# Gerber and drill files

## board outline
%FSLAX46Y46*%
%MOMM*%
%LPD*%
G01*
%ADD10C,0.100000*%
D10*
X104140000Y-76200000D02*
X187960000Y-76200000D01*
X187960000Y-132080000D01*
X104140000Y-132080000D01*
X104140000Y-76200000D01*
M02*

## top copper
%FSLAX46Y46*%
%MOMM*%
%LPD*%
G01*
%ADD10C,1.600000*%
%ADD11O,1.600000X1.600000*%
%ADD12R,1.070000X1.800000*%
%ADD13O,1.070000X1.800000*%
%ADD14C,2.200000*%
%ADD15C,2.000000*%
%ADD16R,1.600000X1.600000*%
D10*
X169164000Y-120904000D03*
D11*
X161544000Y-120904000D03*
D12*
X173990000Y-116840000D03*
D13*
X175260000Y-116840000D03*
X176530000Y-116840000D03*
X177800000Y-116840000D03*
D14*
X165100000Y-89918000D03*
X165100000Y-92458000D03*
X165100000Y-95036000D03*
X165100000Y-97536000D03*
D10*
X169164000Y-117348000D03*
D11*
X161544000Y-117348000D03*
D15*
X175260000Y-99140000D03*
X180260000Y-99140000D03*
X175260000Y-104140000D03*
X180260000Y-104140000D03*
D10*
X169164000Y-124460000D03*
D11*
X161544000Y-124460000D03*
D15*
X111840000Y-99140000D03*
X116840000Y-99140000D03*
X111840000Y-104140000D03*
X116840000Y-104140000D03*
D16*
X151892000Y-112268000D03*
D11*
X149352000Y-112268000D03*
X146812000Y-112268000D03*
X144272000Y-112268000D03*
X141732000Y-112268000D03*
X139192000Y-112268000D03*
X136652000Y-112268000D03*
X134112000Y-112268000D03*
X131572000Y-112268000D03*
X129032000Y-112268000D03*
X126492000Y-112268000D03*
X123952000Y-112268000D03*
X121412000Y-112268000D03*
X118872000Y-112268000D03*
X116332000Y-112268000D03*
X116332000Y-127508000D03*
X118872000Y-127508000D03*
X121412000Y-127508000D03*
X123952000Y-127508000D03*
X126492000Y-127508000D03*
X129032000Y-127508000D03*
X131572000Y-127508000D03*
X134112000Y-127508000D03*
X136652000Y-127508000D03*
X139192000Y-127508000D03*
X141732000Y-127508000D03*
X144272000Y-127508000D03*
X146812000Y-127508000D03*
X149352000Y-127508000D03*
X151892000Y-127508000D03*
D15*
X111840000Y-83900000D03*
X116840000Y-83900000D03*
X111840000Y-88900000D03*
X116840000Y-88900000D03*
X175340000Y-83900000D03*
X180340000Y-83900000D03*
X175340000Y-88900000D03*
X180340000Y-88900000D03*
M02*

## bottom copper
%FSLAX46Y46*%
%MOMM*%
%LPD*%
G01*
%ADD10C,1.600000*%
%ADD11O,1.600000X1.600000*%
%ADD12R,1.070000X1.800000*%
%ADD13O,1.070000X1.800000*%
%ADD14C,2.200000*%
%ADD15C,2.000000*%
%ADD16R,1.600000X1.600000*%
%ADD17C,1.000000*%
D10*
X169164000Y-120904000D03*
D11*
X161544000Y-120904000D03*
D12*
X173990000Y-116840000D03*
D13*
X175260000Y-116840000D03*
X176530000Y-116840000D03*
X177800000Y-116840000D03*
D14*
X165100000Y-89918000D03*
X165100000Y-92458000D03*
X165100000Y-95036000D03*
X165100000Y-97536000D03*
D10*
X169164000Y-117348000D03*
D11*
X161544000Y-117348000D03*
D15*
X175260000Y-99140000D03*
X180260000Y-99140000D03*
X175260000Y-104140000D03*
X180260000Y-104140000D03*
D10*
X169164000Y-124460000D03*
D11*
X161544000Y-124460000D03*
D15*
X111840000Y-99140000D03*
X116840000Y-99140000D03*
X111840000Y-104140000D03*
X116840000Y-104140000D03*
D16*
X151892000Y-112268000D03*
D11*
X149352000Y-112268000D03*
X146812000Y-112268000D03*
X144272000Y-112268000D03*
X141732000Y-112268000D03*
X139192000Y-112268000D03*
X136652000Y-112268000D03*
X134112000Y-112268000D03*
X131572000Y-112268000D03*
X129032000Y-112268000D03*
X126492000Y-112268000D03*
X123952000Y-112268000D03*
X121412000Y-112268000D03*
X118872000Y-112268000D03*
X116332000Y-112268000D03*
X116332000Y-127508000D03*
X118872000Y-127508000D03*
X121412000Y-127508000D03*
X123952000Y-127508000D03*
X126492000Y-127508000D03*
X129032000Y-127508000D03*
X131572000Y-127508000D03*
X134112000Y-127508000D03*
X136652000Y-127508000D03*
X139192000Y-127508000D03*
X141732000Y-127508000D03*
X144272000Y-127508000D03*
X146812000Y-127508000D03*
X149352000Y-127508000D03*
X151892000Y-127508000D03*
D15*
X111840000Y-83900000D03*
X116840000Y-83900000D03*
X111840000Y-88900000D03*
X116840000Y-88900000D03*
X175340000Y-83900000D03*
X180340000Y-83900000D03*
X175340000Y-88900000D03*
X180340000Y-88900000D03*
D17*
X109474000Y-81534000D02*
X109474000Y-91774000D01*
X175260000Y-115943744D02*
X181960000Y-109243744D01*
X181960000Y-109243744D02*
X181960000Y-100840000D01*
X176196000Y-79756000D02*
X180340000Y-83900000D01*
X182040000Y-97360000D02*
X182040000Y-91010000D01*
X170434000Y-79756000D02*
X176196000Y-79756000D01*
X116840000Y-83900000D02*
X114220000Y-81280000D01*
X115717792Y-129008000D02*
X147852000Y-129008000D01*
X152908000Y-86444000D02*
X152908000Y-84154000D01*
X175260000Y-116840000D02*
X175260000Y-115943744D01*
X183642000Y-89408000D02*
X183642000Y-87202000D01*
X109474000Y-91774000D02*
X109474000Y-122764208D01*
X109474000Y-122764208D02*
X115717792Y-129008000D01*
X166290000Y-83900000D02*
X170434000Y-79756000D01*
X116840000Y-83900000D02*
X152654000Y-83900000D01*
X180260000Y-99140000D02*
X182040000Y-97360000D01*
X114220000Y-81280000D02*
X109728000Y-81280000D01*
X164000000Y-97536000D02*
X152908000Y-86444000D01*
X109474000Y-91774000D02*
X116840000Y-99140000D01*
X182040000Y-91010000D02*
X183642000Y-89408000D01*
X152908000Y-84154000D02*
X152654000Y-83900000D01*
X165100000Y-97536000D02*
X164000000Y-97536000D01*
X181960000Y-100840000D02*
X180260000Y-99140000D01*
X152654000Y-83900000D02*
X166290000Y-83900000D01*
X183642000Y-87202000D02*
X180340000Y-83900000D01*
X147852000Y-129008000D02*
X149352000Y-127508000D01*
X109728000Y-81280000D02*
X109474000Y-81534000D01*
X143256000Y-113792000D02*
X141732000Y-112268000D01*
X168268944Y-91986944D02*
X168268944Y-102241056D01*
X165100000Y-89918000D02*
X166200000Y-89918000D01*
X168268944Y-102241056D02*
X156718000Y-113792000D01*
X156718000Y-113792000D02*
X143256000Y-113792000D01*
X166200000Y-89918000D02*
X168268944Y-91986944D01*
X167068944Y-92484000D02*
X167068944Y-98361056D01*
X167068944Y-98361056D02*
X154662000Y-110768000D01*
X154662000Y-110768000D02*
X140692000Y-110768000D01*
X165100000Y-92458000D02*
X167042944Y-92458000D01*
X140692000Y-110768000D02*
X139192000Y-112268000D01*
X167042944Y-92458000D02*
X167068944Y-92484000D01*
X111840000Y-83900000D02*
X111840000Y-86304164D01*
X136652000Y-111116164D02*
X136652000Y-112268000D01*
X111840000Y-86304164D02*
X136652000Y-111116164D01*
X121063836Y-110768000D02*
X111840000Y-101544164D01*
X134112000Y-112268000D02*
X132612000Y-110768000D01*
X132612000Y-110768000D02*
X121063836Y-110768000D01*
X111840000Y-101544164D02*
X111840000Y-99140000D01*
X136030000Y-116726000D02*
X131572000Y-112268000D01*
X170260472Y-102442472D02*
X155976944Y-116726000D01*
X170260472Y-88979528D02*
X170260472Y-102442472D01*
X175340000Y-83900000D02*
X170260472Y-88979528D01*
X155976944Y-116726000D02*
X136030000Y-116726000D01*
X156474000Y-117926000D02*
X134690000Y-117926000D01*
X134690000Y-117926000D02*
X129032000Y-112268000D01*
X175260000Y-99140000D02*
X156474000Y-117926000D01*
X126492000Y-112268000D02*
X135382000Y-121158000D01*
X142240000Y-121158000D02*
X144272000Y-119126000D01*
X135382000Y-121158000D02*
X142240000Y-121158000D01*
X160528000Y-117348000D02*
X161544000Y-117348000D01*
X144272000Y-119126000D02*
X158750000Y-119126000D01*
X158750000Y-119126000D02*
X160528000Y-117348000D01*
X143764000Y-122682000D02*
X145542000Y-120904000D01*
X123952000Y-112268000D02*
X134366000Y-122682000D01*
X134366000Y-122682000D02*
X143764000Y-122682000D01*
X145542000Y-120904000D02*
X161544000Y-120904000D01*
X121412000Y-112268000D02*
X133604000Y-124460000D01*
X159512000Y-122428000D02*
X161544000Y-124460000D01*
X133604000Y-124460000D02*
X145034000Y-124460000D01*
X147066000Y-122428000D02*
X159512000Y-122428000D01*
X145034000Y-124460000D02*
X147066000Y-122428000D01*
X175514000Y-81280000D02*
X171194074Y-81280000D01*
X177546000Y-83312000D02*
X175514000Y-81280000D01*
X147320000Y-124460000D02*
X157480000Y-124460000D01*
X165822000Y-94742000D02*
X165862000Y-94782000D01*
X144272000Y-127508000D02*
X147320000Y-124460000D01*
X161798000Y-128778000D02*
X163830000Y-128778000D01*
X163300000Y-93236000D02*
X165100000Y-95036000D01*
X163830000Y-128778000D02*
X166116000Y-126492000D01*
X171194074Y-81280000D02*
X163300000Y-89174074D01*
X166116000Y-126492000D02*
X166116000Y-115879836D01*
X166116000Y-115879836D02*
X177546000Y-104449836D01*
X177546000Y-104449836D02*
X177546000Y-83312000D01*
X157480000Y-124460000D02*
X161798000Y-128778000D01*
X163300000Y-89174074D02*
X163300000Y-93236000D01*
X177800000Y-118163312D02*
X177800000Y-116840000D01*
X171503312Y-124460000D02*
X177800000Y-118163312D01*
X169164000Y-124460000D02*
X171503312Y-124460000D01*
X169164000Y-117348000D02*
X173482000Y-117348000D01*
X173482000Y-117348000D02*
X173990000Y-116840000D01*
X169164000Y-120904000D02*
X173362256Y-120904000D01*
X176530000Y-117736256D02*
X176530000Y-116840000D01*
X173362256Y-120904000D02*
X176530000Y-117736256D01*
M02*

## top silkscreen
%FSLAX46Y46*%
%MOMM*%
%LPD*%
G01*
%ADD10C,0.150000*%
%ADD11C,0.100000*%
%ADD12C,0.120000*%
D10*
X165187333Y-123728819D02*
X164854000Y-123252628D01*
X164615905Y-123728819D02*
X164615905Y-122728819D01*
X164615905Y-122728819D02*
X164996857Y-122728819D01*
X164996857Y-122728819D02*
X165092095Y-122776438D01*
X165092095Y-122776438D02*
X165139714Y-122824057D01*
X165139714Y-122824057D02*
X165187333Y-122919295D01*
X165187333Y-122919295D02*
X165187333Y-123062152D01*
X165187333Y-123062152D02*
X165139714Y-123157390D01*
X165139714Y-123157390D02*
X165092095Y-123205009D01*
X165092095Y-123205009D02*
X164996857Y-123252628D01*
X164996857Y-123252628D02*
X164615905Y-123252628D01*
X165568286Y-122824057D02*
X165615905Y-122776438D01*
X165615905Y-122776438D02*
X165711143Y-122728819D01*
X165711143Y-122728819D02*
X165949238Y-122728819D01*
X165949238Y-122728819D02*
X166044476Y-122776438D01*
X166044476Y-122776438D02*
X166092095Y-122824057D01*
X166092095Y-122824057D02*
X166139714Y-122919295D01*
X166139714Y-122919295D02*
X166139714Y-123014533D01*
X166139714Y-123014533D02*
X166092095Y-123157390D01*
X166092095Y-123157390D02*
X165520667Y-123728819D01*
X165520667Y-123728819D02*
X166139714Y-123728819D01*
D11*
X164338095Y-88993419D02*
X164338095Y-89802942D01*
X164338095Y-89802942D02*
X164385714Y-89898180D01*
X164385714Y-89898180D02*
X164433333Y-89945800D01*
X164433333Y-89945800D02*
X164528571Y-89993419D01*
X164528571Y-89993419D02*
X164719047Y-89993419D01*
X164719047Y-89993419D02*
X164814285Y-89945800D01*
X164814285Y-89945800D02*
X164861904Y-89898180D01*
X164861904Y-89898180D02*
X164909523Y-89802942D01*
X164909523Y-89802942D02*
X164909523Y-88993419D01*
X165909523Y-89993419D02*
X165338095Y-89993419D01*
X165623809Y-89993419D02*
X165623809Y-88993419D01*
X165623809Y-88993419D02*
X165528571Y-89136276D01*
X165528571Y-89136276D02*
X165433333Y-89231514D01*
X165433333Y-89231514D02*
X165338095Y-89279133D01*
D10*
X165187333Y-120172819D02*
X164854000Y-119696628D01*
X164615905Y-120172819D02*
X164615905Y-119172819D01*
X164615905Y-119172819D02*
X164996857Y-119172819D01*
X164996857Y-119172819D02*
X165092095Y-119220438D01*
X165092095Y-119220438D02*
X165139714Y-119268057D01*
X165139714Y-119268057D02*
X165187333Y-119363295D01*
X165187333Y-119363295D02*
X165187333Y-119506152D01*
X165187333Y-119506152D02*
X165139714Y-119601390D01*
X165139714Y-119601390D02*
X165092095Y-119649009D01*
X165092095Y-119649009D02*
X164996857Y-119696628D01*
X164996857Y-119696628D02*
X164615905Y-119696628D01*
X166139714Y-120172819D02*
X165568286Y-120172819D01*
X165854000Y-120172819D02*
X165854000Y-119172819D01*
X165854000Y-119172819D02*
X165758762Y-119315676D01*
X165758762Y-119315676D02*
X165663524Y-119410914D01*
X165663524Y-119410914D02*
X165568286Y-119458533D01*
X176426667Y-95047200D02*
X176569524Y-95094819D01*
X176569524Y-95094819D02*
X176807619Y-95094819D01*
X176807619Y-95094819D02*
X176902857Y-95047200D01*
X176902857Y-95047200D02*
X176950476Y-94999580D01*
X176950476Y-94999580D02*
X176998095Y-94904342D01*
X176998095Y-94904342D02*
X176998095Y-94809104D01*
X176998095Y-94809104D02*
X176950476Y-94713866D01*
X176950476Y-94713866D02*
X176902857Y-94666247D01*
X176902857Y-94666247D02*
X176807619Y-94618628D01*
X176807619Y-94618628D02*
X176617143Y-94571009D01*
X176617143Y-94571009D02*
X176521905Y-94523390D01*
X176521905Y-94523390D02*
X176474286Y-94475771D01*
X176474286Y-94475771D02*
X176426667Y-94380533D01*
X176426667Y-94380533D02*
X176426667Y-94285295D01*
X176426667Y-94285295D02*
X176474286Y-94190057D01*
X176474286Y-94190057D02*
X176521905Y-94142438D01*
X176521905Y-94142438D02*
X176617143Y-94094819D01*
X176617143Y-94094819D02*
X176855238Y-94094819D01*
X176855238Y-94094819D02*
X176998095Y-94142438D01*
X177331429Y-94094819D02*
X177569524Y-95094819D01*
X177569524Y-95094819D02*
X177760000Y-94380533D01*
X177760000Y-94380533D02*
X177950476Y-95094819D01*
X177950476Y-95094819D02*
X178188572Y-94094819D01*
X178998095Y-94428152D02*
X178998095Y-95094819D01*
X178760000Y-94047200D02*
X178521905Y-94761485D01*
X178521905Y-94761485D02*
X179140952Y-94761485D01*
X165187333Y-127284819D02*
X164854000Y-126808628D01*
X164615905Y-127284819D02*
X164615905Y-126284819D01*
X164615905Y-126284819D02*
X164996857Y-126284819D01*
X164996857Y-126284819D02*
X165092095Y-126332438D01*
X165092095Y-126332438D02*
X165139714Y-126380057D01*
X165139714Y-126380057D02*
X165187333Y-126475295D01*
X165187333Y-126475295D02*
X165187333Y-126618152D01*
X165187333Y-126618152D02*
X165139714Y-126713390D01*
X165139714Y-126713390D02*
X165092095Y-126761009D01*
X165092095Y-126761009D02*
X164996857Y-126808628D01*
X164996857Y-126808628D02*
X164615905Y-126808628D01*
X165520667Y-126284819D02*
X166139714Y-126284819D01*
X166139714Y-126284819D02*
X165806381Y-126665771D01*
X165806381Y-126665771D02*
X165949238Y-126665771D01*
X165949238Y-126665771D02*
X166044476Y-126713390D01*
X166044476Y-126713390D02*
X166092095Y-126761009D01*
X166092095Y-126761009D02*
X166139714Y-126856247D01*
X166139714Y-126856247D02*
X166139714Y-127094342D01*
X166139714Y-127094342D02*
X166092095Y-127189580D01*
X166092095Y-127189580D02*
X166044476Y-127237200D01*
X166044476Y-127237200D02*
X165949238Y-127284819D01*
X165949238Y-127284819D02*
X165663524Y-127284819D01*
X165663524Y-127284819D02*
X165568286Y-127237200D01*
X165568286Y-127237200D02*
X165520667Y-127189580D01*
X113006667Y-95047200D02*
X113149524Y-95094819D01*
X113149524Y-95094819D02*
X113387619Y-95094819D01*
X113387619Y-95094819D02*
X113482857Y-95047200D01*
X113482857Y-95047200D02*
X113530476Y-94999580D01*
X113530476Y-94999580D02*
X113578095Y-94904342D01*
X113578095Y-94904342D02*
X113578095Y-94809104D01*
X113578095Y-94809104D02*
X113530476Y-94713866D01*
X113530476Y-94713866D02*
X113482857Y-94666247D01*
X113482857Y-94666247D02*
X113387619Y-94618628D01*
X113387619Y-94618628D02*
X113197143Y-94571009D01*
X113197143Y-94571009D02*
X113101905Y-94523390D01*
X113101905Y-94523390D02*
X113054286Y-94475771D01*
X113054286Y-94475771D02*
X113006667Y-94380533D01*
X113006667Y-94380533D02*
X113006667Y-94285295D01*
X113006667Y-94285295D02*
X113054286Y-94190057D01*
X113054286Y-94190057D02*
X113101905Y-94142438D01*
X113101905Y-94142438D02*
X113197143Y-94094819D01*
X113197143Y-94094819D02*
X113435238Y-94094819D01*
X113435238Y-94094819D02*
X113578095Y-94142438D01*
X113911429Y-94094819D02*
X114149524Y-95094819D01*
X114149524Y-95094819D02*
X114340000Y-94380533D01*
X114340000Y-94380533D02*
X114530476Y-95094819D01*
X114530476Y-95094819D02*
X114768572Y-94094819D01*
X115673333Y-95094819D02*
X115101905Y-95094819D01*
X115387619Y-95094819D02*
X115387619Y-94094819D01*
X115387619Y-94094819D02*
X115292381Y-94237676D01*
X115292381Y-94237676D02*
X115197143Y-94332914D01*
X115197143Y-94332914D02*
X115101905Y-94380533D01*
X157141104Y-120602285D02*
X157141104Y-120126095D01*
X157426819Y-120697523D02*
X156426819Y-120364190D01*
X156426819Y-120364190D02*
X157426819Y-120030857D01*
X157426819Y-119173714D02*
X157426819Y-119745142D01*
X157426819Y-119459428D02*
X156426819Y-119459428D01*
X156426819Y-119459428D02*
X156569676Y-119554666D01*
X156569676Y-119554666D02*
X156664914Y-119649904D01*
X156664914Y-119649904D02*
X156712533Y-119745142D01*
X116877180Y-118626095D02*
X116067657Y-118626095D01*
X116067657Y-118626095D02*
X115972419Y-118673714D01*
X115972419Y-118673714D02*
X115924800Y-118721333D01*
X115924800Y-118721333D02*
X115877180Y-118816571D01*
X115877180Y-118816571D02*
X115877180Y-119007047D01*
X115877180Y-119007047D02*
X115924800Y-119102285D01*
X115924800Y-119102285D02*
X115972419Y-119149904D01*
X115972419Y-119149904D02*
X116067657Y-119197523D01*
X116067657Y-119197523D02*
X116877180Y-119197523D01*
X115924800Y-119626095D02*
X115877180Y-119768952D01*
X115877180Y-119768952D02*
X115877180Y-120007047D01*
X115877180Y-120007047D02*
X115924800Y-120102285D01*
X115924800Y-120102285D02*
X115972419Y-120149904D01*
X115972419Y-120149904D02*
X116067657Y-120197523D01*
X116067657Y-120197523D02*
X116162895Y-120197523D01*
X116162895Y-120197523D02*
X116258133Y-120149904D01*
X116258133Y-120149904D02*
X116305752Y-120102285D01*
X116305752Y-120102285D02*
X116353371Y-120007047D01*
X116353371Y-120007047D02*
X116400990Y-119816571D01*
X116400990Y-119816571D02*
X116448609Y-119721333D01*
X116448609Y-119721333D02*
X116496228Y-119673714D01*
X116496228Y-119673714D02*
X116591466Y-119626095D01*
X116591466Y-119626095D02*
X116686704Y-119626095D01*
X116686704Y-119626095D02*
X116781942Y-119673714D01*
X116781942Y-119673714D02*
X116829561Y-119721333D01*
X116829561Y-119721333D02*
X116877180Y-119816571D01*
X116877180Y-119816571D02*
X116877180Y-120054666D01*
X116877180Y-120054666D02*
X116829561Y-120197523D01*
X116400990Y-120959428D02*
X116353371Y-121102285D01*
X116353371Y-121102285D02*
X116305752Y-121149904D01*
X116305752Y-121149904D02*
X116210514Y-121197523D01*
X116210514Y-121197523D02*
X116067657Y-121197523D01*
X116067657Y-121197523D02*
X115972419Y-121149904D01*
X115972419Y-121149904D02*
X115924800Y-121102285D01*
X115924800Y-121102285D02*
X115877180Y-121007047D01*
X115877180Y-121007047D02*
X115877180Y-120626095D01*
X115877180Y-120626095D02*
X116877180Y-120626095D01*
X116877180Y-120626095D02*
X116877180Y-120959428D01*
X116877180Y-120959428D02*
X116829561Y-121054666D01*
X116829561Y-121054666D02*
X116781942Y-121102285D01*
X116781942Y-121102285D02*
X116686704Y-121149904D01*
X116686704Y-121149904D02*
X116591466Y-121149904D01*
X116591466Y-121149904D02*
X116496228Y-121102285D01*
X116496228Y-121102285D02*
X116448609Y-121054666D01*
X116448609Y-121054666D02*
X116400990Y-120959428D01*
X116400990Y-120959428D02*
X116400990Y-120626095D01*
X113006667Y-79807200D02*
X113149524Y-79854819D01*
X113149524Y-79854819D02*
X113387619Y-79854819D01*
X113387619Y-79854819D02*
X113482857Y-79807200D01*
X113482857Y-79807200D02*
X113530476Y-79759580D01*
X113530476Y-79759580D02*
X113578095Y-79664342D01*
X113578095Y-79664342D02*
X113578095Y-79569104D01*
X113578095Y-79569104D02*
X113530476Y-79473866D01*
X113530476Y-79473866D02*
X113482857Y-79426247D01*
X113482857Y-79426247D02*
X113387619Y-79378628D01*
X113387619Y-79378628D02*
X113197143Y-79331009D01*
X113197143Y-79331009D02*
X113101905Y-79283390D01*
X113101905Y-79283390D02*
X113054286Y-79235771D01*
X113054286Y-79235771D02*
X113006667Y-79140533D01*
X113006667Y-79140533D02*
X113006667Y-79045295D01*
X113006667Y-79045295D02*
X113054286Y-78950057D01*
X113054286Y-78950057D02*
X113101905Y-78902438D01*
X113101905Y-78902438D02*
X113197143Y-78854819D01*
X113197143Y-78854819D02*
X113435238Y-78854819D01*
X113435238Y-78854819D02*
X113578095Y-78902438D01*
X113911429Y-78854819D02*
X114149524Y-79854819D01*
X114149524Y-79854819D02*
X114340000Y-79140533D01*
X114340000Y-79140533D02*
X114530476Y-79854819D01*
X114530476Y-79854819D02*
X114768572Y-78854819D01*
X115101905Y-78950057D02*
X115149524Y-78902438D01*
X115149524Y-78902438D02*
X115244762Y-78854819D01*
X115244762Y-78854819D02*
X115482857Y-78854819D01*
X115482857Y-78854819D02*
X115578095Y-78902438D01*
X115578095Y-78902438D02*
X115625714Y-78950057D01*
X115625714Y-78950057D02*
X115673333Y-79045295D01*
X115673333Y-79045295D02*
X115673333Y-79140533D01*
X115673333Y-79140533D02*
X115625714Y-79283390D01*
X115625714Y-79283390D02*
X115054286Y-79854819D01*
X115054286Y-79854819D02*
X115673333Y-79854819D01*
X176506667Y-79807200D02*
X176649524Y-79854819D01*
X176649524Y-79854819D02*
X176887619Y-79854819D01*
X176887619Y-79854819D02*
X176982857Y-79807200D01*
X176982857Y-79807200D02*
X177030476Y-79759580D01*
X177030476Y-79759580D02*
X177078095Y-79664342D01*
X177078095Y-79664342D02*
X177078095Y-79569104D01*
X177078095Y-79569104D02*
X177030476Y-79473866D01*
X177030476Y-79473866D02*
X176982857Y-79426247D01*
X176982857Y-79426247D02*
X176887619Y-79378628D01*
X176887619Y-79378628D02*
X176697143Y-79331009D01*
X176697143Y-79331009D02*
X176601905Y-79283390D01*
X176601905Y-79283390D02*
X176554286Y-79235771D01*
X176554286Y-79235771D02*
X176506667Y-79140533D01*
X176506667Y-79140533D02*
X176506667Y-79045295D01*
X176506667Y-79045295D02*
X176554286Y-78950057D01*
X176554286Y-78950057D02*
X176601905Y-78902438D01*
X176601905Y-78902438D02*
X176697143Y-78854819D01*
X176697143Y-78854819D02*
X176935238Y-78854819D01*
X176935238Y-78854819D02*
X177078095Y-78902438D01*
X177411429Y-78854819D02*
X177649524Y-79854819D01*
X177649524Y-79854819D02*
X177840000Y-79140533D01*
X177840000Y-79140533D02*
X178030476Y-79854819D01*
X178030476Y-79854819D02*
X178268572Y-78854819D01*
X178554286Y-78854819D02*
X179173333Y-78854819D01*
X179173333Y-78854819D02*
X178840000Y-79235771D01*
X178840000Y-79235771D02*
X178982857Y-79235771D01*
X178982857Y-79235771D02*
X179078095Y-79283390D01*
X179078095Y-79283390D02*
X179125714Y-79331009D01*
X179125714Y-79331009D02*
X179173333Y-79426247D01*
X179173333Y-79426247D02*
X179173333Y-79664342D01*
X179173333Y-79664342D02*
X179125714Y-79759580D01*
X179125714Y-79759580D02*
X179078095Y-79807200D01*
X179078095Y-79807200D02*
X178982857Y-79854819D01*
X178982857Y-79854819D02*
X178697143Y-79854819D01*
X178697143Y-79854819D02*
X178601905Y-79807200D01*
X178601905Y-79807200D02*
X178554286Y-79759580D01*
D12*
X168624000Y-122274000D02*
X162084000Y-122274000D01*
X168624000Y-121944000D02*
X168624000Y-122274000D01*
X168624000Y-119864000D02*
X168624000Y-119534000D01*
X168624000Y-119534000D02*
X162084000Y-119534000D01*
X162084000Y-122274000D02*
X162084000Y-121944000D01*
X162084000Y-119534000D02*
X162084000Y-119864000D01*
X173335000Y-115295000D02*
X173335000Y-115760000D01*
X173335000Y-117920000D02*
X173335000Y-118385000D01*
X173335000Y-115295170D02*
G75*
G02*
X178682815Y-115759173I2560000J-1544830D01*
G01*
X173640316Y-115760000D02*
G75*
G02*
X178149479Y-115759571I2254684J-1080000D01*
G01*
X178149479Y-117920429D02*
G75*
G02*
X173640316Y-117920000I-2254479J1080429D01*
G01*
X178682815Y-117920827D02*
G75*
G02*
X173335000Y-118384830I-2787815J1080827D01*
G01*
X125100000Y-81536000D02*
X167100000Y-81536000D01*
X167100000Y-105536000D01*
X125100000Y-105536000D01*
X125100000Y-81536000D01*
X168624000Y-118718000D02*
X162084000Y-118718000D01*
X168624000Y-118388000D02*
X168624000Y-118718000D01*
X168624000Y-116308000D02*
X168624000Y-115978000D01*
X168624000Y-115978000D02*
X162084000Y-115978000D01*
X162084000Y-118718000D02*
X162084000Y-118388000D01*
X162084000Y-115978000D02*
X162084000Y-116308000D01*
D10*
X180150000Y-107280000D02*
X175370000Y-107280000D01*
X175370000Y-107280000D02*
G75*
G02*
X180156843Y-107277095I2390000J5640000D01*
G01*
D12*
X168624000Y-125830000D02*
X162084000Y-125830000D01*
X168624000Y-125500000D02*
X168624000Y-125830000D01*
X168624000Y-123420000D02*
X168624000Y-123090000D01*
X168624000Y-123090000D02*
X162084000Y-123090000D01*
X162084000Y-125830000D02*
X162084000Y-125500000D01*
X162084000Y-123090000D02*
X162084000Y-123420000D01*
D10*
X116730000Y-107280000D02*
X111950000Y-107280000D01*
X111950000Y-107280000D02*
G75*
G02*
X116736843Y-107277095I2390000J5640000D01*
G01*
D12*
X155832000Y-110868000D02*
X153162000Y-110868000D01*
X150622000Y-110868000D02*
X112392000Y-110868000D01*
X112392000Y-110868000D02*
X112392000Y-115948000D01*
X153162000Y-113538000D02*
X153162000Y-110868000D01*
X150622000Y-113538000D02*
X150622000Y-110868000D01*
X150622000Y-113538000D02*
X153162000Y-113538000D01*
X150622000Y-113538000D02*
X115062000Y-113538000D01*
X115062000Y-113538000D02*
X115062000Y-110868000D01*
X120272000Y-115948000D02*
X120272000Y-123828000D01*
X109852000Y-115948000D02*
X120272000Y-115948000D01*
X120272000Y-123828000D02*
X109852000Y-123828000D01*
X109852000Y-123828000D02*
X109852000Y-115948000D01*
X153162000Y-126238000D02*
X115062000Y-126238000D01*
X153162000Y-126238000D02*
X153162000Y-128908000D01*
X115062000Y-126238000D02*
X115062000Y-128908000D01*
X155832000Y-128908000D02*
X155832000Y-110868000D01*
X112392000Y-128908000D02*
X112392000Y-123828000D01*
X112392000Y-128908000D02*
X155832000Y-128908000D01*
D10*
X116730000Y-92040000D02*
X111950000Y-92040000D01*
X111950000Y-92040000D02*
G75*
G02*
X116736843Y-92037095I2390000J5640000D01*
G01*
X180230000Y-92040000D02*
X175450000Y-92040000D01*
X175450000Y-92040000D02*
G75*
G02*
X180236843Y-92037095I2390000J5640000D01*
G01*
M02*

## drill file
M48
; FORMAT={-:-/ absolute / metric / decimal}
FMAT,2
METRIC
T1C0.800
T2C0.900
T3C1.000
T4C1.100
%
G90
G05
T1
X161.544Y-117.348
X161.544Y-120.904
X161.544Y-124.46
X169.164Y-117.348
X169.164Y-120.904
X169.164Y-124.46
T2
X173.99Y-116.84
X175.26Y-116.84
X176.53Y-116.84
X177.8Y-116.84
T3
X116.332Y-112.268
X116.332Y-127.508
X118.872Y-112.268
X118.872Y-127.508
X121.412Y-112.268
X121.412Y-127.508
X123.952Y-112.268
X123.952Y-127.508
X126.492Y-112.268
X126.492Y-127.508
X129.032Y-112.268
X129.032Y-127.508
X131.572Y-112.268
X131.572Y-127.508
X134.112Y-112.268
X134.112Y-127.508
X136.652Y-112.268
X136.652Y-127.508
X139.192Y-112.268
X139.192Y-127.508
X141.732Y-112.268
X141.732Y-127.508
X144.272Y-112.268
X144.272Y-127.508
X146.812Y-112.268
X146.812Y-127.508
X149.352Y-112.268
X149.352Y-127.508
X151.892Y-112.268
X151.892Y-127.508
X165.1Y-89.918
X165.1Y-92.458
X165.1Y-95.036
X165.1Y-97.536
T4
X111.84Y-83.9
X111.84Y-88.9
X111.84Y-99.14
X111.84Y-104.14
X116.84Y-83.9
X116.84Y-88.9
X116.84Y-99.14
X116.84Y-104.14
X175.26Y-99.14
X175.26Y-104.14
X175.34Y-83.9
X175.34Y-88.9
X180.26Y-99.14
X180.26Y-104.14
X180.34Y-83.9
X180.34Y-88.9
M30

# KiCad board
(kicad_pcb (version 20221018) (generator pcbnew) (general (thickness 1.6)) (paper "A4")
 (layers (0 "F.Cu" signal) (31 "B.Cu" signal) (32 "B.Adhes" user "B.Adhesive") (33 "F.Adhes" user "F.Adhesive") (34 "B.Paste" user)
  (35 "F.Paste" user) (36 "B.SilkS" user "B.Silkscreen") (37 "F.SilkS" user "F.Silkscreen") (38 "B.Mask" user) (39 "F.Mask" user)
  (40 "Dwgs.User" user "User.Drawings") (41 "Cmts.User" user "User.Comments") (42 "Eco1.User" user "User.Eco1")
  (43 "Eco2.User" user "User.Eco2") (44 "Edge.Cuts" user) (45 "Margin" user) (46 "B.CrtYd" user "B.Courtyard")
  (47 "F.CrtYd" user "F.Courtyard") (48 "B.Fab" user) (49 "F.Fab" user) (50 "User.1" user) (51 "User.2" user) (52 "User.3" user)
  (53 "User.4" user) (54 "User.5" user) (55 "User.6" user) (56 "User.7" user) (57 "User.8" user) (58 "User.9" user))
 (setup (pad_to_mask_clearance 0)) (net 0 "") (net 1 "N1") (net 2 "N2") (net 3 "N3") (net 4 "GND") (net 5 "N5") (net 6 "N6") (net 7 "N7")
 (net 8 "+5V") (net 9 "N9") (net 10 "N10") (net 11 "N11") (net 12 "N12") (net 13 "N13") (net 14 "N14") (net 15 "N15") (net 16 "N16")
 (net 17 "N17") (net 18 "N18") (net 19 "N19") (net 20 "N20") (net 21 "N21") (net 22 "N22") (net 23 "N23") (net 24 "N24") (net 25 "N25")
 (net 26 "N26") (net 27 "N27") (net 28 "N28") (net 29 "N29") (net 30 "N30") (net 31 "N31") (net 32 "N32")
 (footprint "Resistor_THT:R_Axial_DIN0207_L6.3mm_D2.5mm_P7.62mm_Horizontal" (layer "F.Cu") (at 169.164 120.904 180)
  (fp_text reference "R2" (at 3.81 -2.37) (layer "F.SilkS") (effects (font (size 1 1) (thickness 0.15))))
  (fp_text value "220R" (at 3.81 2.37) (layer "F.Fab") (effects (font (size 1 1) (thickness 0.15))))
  (fp_line (start 0.54 -1.37) (end 7.08 -1.37) (stroke (width 0.12) (type solid)) (layer "F.SilkS"))
  (fp_line (start 0.54 -1.04) (end 0.54 -1.37) (stroke (width 0.12) (type solid)) (layer "F.SilkS"))
  (fp_line (start 0.54 1.04) (end 0.54 1.37) (stroke (width 0.12) (type solid)) (layer "F.SilkS"))
  (fp_line (start 0.54 1.37) (end 7.08 1.37) (stroke (width 0.12) (type solid)) (layer "F.SilkS"))
  (fp_line (start 7.08 -1.37) (end 7.08 -1.04) (stroke (width 0.12) (type solid)) (layer "F.SilkS"))
  (fp_line (start 7.08 1.37) (end 7.08 1.04) (stroke (width 0.12) (type solid)) (layer "F.SilkS"))
  (pad "1" thru_hole circle (at 0 0 180) (size 1.6 1.6) (drill 0.8) (layers "*.Cu" "*.Mask") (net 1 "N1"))
  (pad "2" thru_hole oval (at 7.62 0 180) (size 1.6 1.6) (drill 0.8) (layers "*.Cu" "*.Mask") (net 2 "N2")))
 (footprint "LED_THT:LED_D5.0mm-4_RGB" (layer "F.Cu") (at 173.99 116.84)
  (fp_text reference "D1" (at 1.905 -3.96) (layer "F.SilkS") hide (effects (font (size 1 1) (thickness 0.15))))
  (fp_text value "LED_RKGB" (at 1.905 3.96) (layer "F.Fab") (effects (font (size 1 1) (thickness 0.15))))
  (fp_line (start -0.655 -1.545) (end -0.655 -1.08) (stroke (width 0.12) (type solid)) (layer "F.SilkS"))
  (fp_line (start -0.655 1.08) (end -0.655 1.545) (stroke (width 0.12) (type solid)) (layer "F.SilkS"))
  (fp_arc (start -0.655 -1.54483) (mid 2.163456 -2.978809) (end 4.692815 -1.080827) (stroke (width 0.12) (type solid)) (layer "F.SilkS"))
  (fp_arc (start -0.349684 -1.08) (mid 1.904762 -2.5) (end 4.159479 -1.080429) (stroke (width 0.12) (type solid)) (layer "F.SilkS"))
  (fp_arc (start 4.159479 1.080429) (mid 1.904762 2.5) (end -0.349684 1.08) (stroke (width 0.12) (type solid)) (layer "F.SilkS"))
  (fp_arc (start 4.692815 1.080827) (mid 2.163456 2.978808) (end -0.655 1.54483) (stroke (width 0.12) (type solid)) (layer "F.SilkS"))
  (pad "1" thru_hole rect (at 0 0) (size 1.07 1.8) (drill 0.9) (layers "*.Cu" "*.Mask") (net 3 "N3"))
  (pad "2" thru_hole oval (at 1.27 0) (size 1.07 1.8) (drill 0.9) (layers "*.Cu" "*.Mask") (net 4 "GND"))
  (pad "3" thru_hole oval (at 2.54 0) (size 1.07 1.8) (drill 0.9) (layers "*.Cu" "*.Mask") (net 1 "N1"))
  (pad "4" thru_hole oval (at 3.81 0) (size 1.07 1.8) (drill 0.9) (layers "*.Cu" "*.Mask") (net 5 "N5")))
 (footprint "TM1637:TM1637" (layer "F.Cu") (at 167.1 81.536)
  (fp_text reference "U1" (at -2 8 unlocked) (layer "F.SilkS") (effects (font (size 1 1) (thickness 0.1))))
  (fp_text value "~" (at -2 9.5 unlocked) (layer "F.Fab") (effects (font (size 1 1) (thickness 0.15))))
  (fp_rect (start 0 0) (end -42 24) (stroke (width 0.12) (type solid)) (fill none) (layer "F.SilkS"))
  (pad "1" thru_hole circle (at -2 8.382) (size 2.2 2.2) (drill 1) (layers "*.Cu" "*.Mask") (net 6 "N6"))
  (pad "2" thru_hole circle (at -2 10.922) (size 2.2 2.2) (drill 1) (layers "*.Cu" "*.Mask") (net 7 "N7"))
  (pad "3" thru_hole circle (at -2 13.5) (size 2.2 2.2) (drill 1) (layers "*.Cu" "*.Mask") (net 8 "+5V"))
  (pad "4" thru_hole circle (at -2 16) (size 2.2 2.2) (drill 1) (layers "*.Cu" "*.Mask") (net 4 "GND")))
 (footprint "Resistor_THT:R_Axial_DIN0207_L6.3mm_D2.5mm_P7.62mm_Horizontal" (layer "F.Cu") (at 169.164 117.348 180)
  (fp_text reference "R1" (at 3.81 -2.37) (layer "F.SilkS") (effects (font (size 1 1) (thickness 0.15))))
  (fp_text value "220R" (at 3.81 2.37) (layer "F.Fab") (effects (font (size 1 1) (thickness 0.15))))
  (fp_line (start 0.54 -1.37) (end 7.08 -1.37) (stroke (width 0.12) (type solid)) (layer "F.SilkS"))
  (fp_line (start 0.54 -1.04) (end 0.54 -1.37) (stroke (width 0.12) (type solid)) (layer "F.SilkS"))
  (fp_line (start 0.54 1.04) (end 0.54 1.37) (stroke (width 0.12) (type solid)) (layer "F.SilkS"))
  (fp_line (start 0.54 1.37) (end 7.08 1.37) (stroke (width 0.12) (type solid)) (layer "F.SilkS"))
  (fp_line (start 7.08 -1.37) (end 7.08 -1.04) (stroke (width 0.12) (type solid)) (layer "F.SilkS"))
  (fp_line (start 7.08 1.37) (end 7.08 1.04) (stroke (width 0.12) (type solid)) (layer "F.SilkS"))
  (pad "1" thru_hole circle (at 0 0 180) (size 1.6 1.6) (drill 0.8) (layers "*.Cu" "*.Mask") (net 3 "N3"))
  (pad "2" thru_hole oval (at 7.62 0 180) (size 1.6 1.6) (drill 0.8) (layers "*.Cu" "*.Mask") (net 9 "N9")))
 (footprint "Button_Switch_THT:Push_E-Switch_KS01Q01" (layer "F.Cu") (at 175.26 99.14)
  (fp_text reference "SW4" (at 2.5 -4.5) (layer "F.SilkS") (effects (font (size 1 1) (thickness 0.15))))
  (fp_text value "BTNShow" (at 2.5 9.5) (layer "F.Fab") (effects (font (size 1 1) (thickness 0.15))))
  (fp_line (start 4.89 8.14) (end 0.11 8.14) (stroke (width 0.15) (type solid)) (layer "F.SilkS"))
  (fp_arc (start 0.11 8.14) (mid 2.496283 -3.625495) (end 4.896843 8.137095) (stroke (width 0.15) (type solid)) (layer "F.SilkS"))
  (pad "1" thru_hole circle (at 0 0) (size 2 2) (drill 1.1) (layers "*.Cu" "*.Mask") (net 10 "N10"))
  (pad "2" thru_hole circle (at 5 0) (size 2 2) (drill 1.1) (layers "*.Cu" "*.Mask") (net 4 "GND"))
  (pad "3" thru_hole circle (at 0 5) (size 2 2) (drill 1.1) (layers "*.Cu" "*.Mask"))
  (pad "4" thru_hole circle (at 5 5) (size 2 2) (drill 1.1) (layers "*.Cu" "*.Mask")))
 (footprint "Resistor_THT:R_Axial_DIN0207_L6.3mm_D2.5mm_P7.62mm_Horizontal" (layer "F.Cu") (at 169.164 124.46 180)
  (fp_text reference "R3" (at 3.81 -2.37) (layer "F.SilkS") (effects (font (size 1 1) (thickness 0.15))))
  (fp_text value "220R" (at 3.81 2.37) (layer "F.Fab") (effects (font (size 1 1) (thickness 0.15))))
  (fp_line (start 0.54 -1.37) (end 7.08 -1.37) (stroke (width 0.12) (type solid)) (layer "F.SilkS"))
  (fp_line (start 0.54 -1.04) (end 0.54 -1.37) (stroke (width 0.12) (type solid)) (layer "F.SilkS"))
  (fp_line (start 0.54 1.04) (end 0.54 1.37) (stroke (width 0.12) (type solid)) (layer "F.SilkS"))
  (fp_line (start 0.54 1.37) (end 7.08 1.37) (stroke (width 0.12) (type solid)) (layer "F.SilkS"))
  (fp_line (start 7.08 -1.37) (end 7.08 -1.04) (stroke (width 0.12) (type solid)) (layer "F.SilkS"))
  (fp_line (start 7.08 1.37) (end 7.08 1.04) (stroke (width 0.12) (type solid)) (layer "F.SilkS"))
  (pad "1" thru_hole circle (at 0 0 180) (size 1.6 1.6) (drill 0.8) (layers "*.Cu" "*.Mask") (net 5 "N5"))
  (pad "2" thru_hole oval (at 7.62 0 180) (size 1.6 1.6) (drill 0.8) (layers "*.Cu" "*.Mask") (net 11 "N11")))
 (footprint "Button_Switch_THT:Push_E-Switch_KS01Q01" (layer "F.Cu") (at 111.84 99.14)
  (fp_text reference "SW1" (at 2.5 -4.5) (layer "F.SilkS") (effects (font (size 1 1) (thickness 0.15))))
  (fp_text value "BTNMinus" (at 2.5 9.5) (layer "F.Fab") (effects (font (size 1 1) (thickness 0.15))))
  (fp_line (start 4.89 8.14) (end 0.11 8.14) (stroke (width 0.15) (type solid)) (layer "F.SilkS"))
  (fp_arc (start 0.11 8.14) (mid 2.496283 -3.625495) (end 4.896843 8.137095) (stroke (width 0.15) (type solid)) (layer "F.SilkS"))
  (pad "1" thru_hole circle (at 0 0) (size 2 2) (drill 1.1) (layers "*.Cu" "*.Mask") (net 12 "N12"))
  (pad "2" thru_hole circle (at 5 0) (size 2 2) (drill 1.1) (layers "*.Cu" "*.Mask") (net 4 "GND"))
  (pad "3" thru_hole circle (at 0 5) (size 2 2) (drill 1.1) (layers "*.Cu" "*.Mask"))
  (pad "4" thru_hole circle (at 5 5) (size 2 2) (drill 1.1) (layers "*.Cu" "*.Mask")))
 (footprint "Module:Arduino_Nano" (layer "F.Cu") (at 151.892 112.268 -90)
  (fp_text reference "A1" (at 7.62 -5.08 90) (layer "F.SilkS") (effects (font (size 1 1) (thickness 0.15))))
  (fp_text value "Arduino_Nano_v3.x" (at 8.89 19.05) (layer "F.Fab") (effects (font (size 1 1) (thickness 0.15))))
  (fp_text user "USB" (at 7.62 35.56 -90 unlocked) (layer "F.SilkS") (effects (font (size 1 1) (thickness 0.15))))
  (fp_line (start -1.4 -3.94) (end -1.4 -1.27) (stroke (width 0.12) (type solid)) (layer "F.SilkS"))
  (fp_line (start -1.4 1.27) (end -1.4 39.5) (stroke (width 0.12) (type solid)) (layer "F.SilkS"))
  (fp_line (start -1.4 39.5) (end 3.68 39.5) (stroke (width 0.12) (type solid)) (layer "F.SilkS"))
  (fp_line (start 1.27 -1.27) (end -1.4 -1.27) (stroke (width 0.12) (type solid)) (layer "F.SilkS"))
  (fp_line (start 1.27 1.27) (end -1.4 1.27) (stroke (width 0.12) (type solid)) (layer "F.SilkS"))
  (fp_line (start 1.27 1.27) (end 1.27 -1.27) (stroke (width 0.12) (type solid)) (layer "F.SilkS"))
  (fp_line (start 1.27 1.27) (end 1.27 36.83) (stroke (width 0.12) (type solid)) (layer "F.SilkS"))
  (fp_line (start 1.27 36.83) (end -1.4 36.83) (stroke (width 0.12) (type solid)) (layer "F.SilkS"))
  (fp_line (start 3.68 31.62) (end 11.56 31.62) (stroke (width 0.12) (type solid)) (layer "F.SilkS"))
  (fp_line (start 3.68 42.04) (end 3.68 31.62) (stroke (width 0.12) (type solid)) (layer "F.SilkS"))
  (fp_line (start 11.56 31.62) (end 11.56 42.04) (stroke (width 0.12) (type solid)) (layer "F.SilkS"))
  (fp_line (start 11.56 42.04) (end 3.68 42.04) (stroke (width 0.12) (type solid)) (layer "F.SilkS"))
  (fp_line (start 13.97 -1.27) (end 13.97 36.83) (stroke (width 0.12) (type solid)) (layer "F.SilkS"))
  (fp_line (start 13.97 -1.27) (end 16.64 -1.27) (stroke (width 0.12) (type solid)) (layer "F.SilkS"))
  (fp_line (start 13.97 36.83) (end 16.64 36.83) (stroke (width 0.12) (type solid)) (layer "F.SilkS"))
  (fp_line (start 16.64 -3.94) (end -1.4 -3.94) (stroke (width 0.12) (type solid)) (layer "F.SilkS"))
  (fp_line (start 16.64 39.5) (end 11.56 39.5) (stroke (width 0.12) (type solid)) (layer "F.SilkS"))
  (fp_line (start 16.64 39.5) (end 16.64 -3.94) (stroke (width 0.12) (type solid)) (layer "F.SilkS"))
  (pad "1" thru_hole rect (at 0 0 270) (size 1.6 1.6) (drill 1) (layers "*.Cu" "*.Mask") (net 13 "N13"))
  (pad "2" thru_hole oval (at 0 2.54 270) (size 1.6 1.6) (drill 1) (layers "*.Cu" "*.Mask") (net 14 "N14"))
  (pad "3" thru_hole oval (at 0 5.08 270) (size 1.6 1.6) (drill 1) (layers "*.Cu" "*.Mask") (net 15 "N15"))
  (pad "4" thru_hole oval (at 0 7.62 270) (size 1.6 1.6) (drill 1) (layers "*.Cu" "*.Mask") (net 4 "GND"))
  (pad "5" thru_hole oval (at 0 10.16 270) (size 1.6 1.6) (drill 1) (layers "*.Cu" "*.Mask") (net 6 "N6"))
  (pad "6" thru_hole oval (at 0 12.7 270) (size 1.6 1.6) (drill 1) (layers "*.Cu" "*.Mask") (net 7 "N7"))
  (pad "7" thru_hole oval (at 0 15.24 270) (size 1.6 1.6) (drill 1) (layers "*.Cu" "*.Mask") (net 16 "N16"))
  (pad "8" thru_hole oval (at 0 17.78 270) (size 1.6 1.6) (drill 1) (layers "*.Cu" "*.Mask") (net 12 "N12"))
  (pad "9" thru_hole oval (at 0 20.32 270) (size 1.6 1.6) (drill 1) (layers "*.Cu" "*.Mask") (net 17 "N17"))
  (pad "10" thru_hole oval (at 0 22.86 270) (size 1.6 1.6) (drill 1) (layers "*.Cu" "*.Mask") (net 10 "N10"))
  (pad "11" thru_hole oval (at 0 25.4 270) (size 1.6 1.6) (drill 1) (layers "*.Cu" "*.Mask") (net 9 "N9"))
  (pad "12" thru_hole oval (at 0 27.94 270) (size 1.6 1.6) (drill 1) (layers "*.Cu" "*.Mask") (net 2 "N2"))
  (pad "13" thru_hole oval (at 0 30.48 270) (size 1.6 1.6) (drill 1) (layers "*.Cu" "*.Mask") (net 11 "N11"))
  (pad "14" thru_hole oval (at 0 33.02 270) (size 1.6 1.6) (drill 1) (layers "*.Cu" "*.Mask") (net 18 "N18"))
  (pad "15" thru_hole oval (at 0 35.56 270) (size 1.6 1.6) (drill 1) (layers "*.Cu" "*.Mask") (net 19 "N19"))
  (pad "16" thru_hole oval (at 15.24 35.56 270) (size 1.6 1.6) (drill 1) (layers "*.Cu" "*.Mask") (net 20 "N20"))
  (pad "17" thru_hole oval (at 15.24 33.02 270) (size 1.6 1.6) (drill 1) (layers "*.Cu" "*.Mask") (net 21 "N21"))
  (pad "18" thru_hole oval (at 15.24 30.48 270) (size 1.6 1.6) (drill 1) (layers "*.Cu" "*.Mask") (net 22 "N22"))
  (pad "19" thru_hole oval (at 15.24 27.94 270) (size 1.6 1.6) (drill 1) (layers "*.Cu" "*.Mask") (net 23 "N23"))
  (pad "20" thru_hole oval (at 15.24 25.4 270) (size 1.6 1.6) (drill 1) (layers "*.Cu" "*.Mask") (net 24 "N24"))
  (pad "21" thru_hole oval (at 15.24 22.86 270) (size 1.6 1.6) (drill 1) (layers "*.Cu" "*.Mask") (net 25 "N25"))
  (pad "22" thru_hole oval (at 15.24 20.32 270) (size 1.6 1.6) (drill 1) (layers "*.Cu" "*.Mask") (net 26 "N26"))
  (pad "23" thru_hole oval (at 15.24 17.78 270) (size 1.6 1.6) (drill 1) (layers "*.Cu" "*.Mask") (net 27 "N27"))
  (pad "24" thru_hole oval (at 15.24 15.24 270) (size 1.6 1.6) (drill 1) (layers "*.Cu" "*.Mask") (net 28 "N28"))
  (pad "25" thru_hole oval (at 15.24 12.7 270) (size 1.6 1.6) (drill 1) (layers "*.Cu" "*.Mask") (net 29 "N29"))
  (pad "26" thru_hole oval (at 15.24 10.16 270) (size 1.6 1.6) (drill 1) (layers "*.Cu" "*.Mask") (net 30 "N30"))
  (pad "27" thru_hole oval (at 15.24 7.62 270) (size 1.6 1.6) (drill 1) (layers "*.Cu" "*.Mask") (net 8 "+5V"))
  (pad "28" thru_hole oval (at 15.24 5.08 270) (size 1.6 1.6) (drill 1) (layers "*.Cu" "*.Mask") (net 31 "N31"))
  (pad "29" thru_hole oval (at 15.24 2.54 270) (size 1.6 1.6) (drill 1) (layers "*.Cu" "*.Mask") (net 4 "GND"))
  (pad "30" thru_hole oval (at 15.24 0 270) (size 1.6 1.6) (drill 1) (layers "*.Cu" "*.Mask") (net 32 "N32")))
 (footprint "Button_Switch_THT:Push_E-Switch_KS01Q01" (layer "F.Cu") (at 111.84 83.9)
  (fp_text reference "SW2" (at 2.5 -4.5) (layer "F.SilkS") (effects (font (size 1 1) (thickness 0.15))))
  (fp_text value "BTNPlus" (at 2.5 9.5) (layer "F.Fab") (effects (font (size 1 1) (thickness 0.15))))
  (fp_line (start 4.89 8.14) (end 0.11 8.14) (stroke (width 0.15) (type solid)) (layer "F.SilkS"))
  (fp_arc (start 0.11 8.14) (mid 2.496283 -3.625495) (end 4.896843 8.137095) (stroke (width 0.15) (type solid)) (layer "F.SilkS"))
  (pad "1" thru_hole circle (at 0 0) (size 2 2) (drill 1.1) (layers "*.Cu" "*.Mask") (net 16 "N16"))
  (pad "2" thru_hole circle (at 5 0) (size 2 2) (drill 1.1) (layers "*.Cu" "*.Mask") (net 4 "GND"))
  (pad "3" thru_hole circle (at 0 5) (size 2 2) (drill 1.1) (layers "*.Cu" "*.Mask"))
  (pad "4" thru_hole circle (at 5 5) (size 2 2) (drill 1.1) (layers "*.Cu" "*.Mask")))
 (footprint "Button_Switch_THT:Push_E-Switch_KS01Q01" (layer "F.Cu") (at 175.34 83.9)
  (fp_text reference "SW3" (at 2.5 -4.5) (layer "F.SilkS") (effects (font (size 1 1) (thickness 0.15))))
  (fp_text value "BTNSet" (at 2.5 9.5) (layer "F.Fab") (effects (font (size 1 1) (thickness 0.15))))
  (fp_line (start 4.89 8.14) (end 0.11 8.14) (stroke (width 0.15) (type solid)) (layer "F.SilkS"))
  (fp_arc (start 0.11 8.14) (mid 2.496283 -3.625495) (end 4.896843 8.137095) (stroke (width 0.15) (type solid)) (layer "F.SilkS"))
  (pad "1" thru_hole circle (at 0 0) (size 2 2) (drill 1.1) (layers "*.Cu" "*.Mask") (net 17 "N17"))
  (pad "2" thru_hole circle (at 5 0) (size 2 2) (drill 1.1) (layers "*.Cu" "*.Mask") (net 4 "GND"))
  (pad "3" thru_hole circle (at 0 5) (size 2 2) (drill 1.1) (layers "*.Cu" "*.Mask"))
  (pad "4" thru_hole circle (at 5 5) (size 2 2) (drill 1.1) (layers "*.Cu" "*.Mask")))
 (gr_rect (start 104.14 76.2) (end 187.96 132.08) (stroke (width 0.1) (type default)) (fill none) (layer "Edge.Cuts"))
 (segment (start 109.474 81.534) (end 109.474 91.774) (width 1) (layer "B.Cu") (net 4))
 (segment (start 175.26 115.943744) (end 181.96 109.243744) (width 1) (layer "B.Cu") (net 4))
 (segment (start 181.96 109.243744) (end 181.96 100.84) (width 1) (layer "B.Cu") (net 4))
 (segment (start 176.196 79.756) (end 180.34 83.9) (width 1) (layer "B.Cu") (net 4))
 (segment (start 182.04 97.36) (end 182.04 91.01) (width 1) (layer "B.Cu") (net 4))
 (segment (start 170.434 79.756) (end 176.196 79.756) (width 1) (layer "B.Cu") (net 4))
 (segment (start 116.84 83.9) (end 114.22 81.28) (width 1) (layer "B.Cu") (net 4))
 (segment (start 115.717792 129.008) (end 147.852 129.008) (width 1) (layer "B.Cu") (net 4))
 (segment (start 152.908 86.444) (end 152.908 84.154) (width 1) (layer "B.Cu") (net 4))
 (segment (start 175.26 116.84) (end 175.26 115.943744) (width 1) (layer "B.Cu") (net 4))
 (segment (start 183.642 89.408) (end 183.642 87.202) (width 1) (layer "B.Cu") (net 4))
 (segment (start 109.474 91.774) (end 109.474 122.764208) (width 1) (layer "B.Cu") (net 4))
 (segment (start 109.474 122.764208) (end 115.717792 129.008) (width 1) (layer "B.Cu") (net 4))
 (segment (start 166.29 83.9) (end 170.434 79.756) (width 1) (layer "B.Cu") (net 4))
 (segment (start 116.84 83.9) (end 152.654 83.9) (width 1) (layer "B.Cu") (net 4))
 (segment (start 180.26 99.14) (end 182.04 97.36) (width 1) (layer "B.Cu") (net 4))
 (segment (start 114.22 81.28) (end 109.728 81.28) (width 1) (layer "B.Cu") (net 4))
 (segment (start 164 97.536) (end 152.908 86.444) (width 1) (layer "B.Cu") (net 4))
 (segment (start 109.474 91.774) (end 116.84 99.14) (width 1) (layer "B.Cu") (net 4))
 (segment (start 182.04 91.01) (end 183.642 89.408) (width 1) (layer "B.Cu") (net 4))
 (segment (start 152.908 84.154) (end 152.654 83.9) (width 1) (layer "B.Cu") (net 4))
 (segment (start 165.1 97.536) (end 164 97.536) (width 1) (layer "B.Cu") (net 4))
 (segment (start 181.96 100.84) (end 180.26 99.14) (width 1) (layer "B.Cu") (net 4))
 (segment (start 152.654 83.9) (end 166.29 83.9) (width 1) (layer "B.Cu") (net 4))
 (segment (start 183.642 87.202) (end 180.34 83.9) (width 1) (layer "B.Cu") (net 4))
 (segment (start 147.852 129.008) (end 149.352 127.508) (width 1) (layer "B.Cu") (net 4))
 (segment (start 109.728 81.28) (end 109.474 81.534) (width 1) (layer "B.Cu") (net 4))
 (segment (start 143.256 113.792) (end 141.732 112.268) (width 1) (layer "B.Cu") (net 6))
 (segment (start 168.268944 91.986944) (end 168.268944 102.241056) (width 1) (layer "B.Cu") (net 6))
 (segment (start 165.1 89.918) (end 166.2 89.918) (width 1) (layer "B.Cu") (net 6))
 (segment (start 168.268944 102.241056) (end 156.718 113.792) (width 1) (layer "B.Cu") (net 6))
 (segment (start 156.718 113.792) (end 143.256 113.792) (width 1) (layer "B.Cu") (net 6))
 (segment (start 166.2 89.918) (end 168.268944 91.986944) (width 1) (layer "B.Cu") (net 6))
 (segment (start 167.068944 92.484) (end 167.068944 98.361056) (width 1) (layer "B.Cu") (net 7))
 (segment (start 167.068944 98.361056) (end 154.662 110.768) (width 1) (layer "B.Cu") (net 7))
 (segment (start 154.662 110.768) (end 140.692 110.768) (width 1) (layer "B.Cu") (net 7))
 (segment (start 165.1 92.458) (end 167.042944 92.458) (width 1) (layer "B.Cu") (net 7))
 (segment (start 140.692 110.768) (end 139.192 112.268) (width 1) (layer "B.Cu") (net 7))
 (segment (start 167.042944 92.458) (end 167.068944 92.484) (width 1) (layer "B.Cu") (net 7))
 (segment (start 111.84 83.9) (end 111.84 86.304164) (width 1) (layer "B.Cu") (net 16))
 (segment (start 136.652 111.116164) (end 136.652 112.268) (width 1) (layer "B.Cu") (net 16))
 (segment (start 111.84 86.304164) (end 136.652 111.116164) (width 1) (layer "B.Cu") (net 16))
 (segment (start 121.063836 110.768) (end 111.84 101.544164) (width 1) (layer "B.Cu") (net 12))
 (segment (start 134.112 112.268) (end 132.612 110.768) (width 1) (layer "B.Cu") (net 12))
 (segment (start 132.612 110.768) (end 121.063836 110.768) (width 1) (layer "B.Cu") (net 12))
 (segment (start 111.84 101.544164) (end 111.84 99.14) (width 1) (layer "B.Cu") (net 12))
 (segment (start 136.03 116.726) (end 131.572 112.268) (width 1) (layer "B.Cu") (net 17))
 (segment (start 170.260472 102.442472) (end 155.976944 116.726) (width 1) (layer "B.Cu") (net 17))
 (segment (start 170.260472 88.979528) (end 170.260472 102.442472) (width 1) (layer "B.Cu") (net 17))
 (segment (start 175.34 83.9) (end 170.260472 88.979528) (width 1) (layer "B.Cu") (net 17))
 (segment (start 155.976944 116.726) (end 136.03 116.726) (width 1) (layer "B.Cu") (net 17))
 (segment (start 156.474 117.926) (end 134.69 117.926) (width 1) (layer "B.Cu") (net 10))
 (segment (start 134.69 117.926) (end 129.032 112.268) (width 1) (layer "B.Cu") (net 10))
 (segment (start 175.26 99.14) (end 156.474 117.926) (width 1) (layer "B.Cu") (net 10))
 (segment (start 126.492 112.268) (end 135.382 121.158) (width 1) (layer "B.Cu") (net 9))
 (segment (start 142.24 121.158) (end 144.272 119.126) (width 1) (layer "B.Cu") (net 9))
 (segment (start 135.382 121.158) (end 142.24 121.158) (width 1) (layer "B.Cu") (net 9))
 (segment (start 160.528 117.348) (end 161.544 117.348) (width 1) (layer "B.Cu") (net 9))
 (segment (start 144.272 119.126) (end 158.75 119.126) (width 1) (layer "B.Cu") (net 9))
 (segment (start 158.75 119.126) (end 160.528 117.348) (width 1) (layer "B.Cu") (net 9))
 (segment (start 143.764 122.682) (end 145.542 120.904) (width 1) (layer "B.Cu") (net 2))
 (segment (start 123.952 112.268) (end 134.366 122.682) (width 1) (layer "B.Cu") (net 2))
 (segment (start 134.366 122.682) (end 143.764 122.682) (width 1) (layer "B.Cu") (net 2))
 (segment (start 145.542 120.904) (end 161.544 120.904) (width 1) (layer "B.Cu") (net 2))
 (segment (start 121.412 112.268) (end 133.604 124.46) (width 1) (layer "B.Cu") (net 11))
 (segment (start 159.512 122.428) (end 161.544 124.46) (width 1) (layer "B.Cu") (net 11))
 (segment (start 133.604 124.46) (end 145.034 124.46) (width 1) (layer "B.Cu") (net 11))
 (segment (start 147.066 122.428) (end 159.512 122.428) (width 1) (layer "B.Cu") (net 11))
 (segment (start 145.034 124.46) (end 147.066 122.428) (width 1) (layer "B.Cu") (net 11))
 (segment (start 175.514 81.28) (end 171.194074 81.28) (width 1) (layer "B.Cu") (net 8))
 (segment (start 177.546 83.312) (end 175.514 81.28) (width 1) (layer "B.Cu") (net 8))
 (segment (start 147.32 124.46) (end 157.48 124.46) (width 1) (layer "B.Cu") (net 8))
 (segment (start 165.822 94.742) (end 165.862 94.782) (width 1) (layer "B.Cu") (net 8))
 (segment (start 144.272 127.508) (end 147.32 124.46) (width 1) (layer "B.Cu") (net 8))
 (segment (start 161.798 128.778) (end 163.83 128.778) (width 1) (layer "B.Cu") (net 8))
 (segment (start 163.3 93.236) (end 165.1 95.036) (width 1) (layer "B.Cu") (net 8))
 (segment (start 163.83 128.778) (end 166.116 126.492) (width 1) (layer "B.Cu") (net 8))
 (segment (start 171.194074 81.28) (end 163.3 89.174074) (width 1) (layer "B.Cu") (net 8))
 (segment (start 166.116 126.492) (end 166.116 115.879836) (width 1) (layer "B.Cu") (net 8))
 (segment (start 166.116 115.879836) (end 177.546 104.449836) (width 1) (layer "B.Cu") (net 8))
 (segment (start 177.546 104.449836) (end 177.546 83.312) (width 1) (layer "B.Cu") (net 8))
 (segment (start 157.48 124.46) (end 161.798 128.778) (width 1) (layer "B.Cu") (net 8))
 (segment (start 163.3 89.174074) (end 163.3 93.236) (width 1) (layer "B.Cu") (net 8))
 (segment (start 177.8 118.163312) (end 177.8 116.84) (width 1) (layer "B.Cu") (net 5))
 (segment (start 171.503312 124.46) (end 177.8 118.163312) (width 1) (layer "B.Cu") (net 5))
 (segment (start 169.164 124.46) (end 171.503312 124.46) (width 1) (layer "B.Cu") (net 5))
 (segment (start 169.164 117.348) (end 173.482 117.348) (width 1) (layer "B.Cu") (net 3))
 (segment (start 173.482 117.348) (end 173.99 116.84) (width 1) (layer "B.Cu") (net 3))
 (segment (start 169.164 120.904) (end 173.362256 120.904) (width 1) (layer "B.Cu") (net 1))
 (segment (start 176.53 117.736256) (end 176.53 116.84) (width 1) (layer "B.Cu") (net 1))
 (segment (start 173.362256 120.904) (end 176.53 117.736256) (width 1) (layer "B.Cu") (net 1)))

